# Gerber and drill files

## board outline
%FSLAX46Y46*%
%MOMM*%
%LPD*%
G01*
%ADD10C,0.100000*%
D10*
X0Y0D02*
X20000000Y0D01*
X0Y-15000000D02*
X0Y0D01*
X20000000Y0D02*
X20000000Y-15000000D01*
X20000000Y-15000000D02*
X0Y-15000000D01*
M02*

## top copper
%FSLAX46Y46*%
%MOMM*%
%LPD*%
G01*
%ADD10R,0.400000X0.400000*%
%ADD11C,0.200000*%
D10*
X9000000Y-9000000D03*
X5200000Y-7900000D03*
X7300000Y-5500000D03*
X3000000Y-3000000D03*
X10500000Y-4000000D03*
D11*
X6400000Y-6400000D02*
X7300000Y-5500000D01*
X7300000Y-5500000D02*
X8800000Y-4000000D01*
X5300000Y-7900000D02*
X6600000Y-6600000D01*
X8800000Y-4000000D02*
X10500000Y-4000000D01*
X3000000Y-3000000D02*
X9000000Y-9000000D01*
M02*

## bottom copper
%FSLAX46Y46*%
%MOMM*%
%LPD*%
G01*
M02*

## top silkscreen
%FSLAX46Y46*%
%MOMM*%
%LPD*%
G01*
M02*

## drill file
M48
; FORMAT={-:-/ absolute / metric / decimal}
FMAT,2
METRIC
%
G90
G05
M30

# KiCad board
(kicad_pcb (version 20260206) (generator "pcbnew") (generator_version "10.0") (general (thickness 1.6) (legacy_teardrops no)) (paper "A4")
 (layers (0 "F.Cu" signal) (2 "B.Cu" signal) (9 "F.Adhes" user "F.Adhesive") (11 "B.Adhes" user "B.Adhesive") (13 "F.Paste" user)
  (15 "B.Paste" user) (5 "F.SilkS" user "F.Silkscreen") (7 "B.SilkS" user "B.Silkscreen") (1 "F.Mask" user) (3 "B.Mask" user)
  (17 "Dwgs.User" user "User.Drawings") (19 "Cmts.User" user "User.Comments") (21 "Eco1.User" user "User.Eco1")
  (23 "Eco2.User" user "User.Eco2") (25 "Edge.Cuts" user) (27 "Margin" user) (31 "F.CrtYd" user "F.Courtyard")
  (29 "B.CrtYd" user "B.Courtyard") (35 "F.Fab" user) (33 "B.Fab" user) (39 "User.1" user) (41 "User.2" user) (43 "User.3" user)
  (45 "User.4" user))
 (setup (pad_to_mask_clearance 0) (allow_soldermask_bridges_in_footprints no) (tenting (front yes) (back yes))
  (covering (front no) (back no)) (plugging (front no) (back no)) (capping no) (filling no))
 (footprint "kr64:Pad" (layer "F.Cu") (at 9 9)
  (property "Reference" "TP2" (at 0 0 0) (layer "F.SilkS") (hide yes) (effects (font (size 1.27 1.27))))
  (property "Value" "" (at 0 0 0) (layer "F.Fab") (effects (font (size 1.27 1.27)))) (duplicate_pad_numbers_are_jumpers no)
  (pad "1" smd rect (at 0 0) (size 0.4 0.4) (layers "F.Cu" "F.Mask" "F.Paste") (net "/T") (thermal_bridge_angle 45)))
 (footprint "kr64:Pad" (layer "F.Cu") (at 5.2 7.9)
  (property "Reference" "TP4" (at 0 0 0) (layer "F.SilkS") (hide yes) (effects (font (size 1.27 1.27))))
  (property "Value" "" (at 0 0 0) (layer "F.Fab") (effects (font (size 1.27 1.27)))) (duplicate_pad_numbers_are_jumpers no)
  (pad "1" smd rect (at 0 0) (size 0.4 0.4) (layers "F.Cu" "F.Mask" "F.Paste") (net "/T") (thermal_bridge_angle 45)))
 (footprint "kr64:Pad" (layer "F.Cu") (at 7.3 5.5)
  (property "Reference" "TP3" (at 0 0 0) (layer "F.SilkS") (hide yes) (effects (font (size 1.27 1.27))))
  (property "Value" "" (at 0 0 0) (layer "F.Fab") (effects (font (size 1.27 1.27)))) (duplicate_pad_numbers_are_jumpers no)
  (pad "1" smd rect (at 0 0) (size 0.4 0.4) (layers "F.Cu" "F.Mask" "F.Paste") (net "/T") (thermal_bridge_angle 45)))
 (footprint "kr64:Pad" (layer "F.Cu") (at 3 3)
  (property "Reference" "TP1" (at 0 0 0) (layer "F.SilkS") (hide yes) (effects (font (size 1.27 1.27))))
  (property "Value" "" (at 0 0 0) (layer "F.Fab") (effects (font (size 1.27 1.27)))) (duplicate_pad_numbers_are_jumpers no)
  (pad "1" smd rect (at 0 0) (size 0.4 0.4) (layers "F.Cu" "F.Mask" "F.Paste") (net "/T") (thermal_bridge_angle 45)))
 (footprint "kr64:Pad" (layer "F.Cu") (at 10.5 4)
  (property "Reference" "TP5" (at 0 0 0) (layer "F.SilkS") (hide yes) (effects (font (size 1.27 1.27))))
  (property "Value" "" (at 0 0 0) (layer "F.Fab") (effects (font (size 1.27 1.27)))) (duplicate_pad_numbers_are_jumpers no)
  (pad "1" smd rect (at 0 0) (size 0.4 0.4) (layers "F.Cu" "F.Mask" "F.Paste") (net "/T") (thermal_bridge_angle 45)))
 (gr_line (start 0 0) (end 20 0) (stroke (width 0.1) (type default)) (layer "Edge.Cuts"))
 (gr_line (start 0 15) (end 0 0) (stroke (width 0.1) (type default)) (layer "Edge.Cuts"))
 (gr_line (start 20 0) (end 20 15) (stroke (width 0.1) (type default)) (layer "Edge.Cuts"))
 (gr_line (start 20 15) (end 0 15) (stroke (width 0.1) (type default)) (layer "Edge.Cuts"))
 (segment (start 6.4 6.4) (end 7.3 5.5) (width 0.2) (layer "F.Cu") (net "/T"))
 (segment (start 7.3 5.5) (end 8.8 4) (width 0.2) (layer "F.Cu") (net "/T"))
 (segment (start 5.3 7.9) (end 6.6 6.6) (width 0.2) (layer "F.Cu") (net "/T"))
 (segment (start 8.8 4) (end 10.5 4) (width 0.2) (layer "F.Cu") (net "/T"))
 (segment (start 3 3) (end 9 9) (width 0.2) (layer "F.Cu") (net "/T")))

